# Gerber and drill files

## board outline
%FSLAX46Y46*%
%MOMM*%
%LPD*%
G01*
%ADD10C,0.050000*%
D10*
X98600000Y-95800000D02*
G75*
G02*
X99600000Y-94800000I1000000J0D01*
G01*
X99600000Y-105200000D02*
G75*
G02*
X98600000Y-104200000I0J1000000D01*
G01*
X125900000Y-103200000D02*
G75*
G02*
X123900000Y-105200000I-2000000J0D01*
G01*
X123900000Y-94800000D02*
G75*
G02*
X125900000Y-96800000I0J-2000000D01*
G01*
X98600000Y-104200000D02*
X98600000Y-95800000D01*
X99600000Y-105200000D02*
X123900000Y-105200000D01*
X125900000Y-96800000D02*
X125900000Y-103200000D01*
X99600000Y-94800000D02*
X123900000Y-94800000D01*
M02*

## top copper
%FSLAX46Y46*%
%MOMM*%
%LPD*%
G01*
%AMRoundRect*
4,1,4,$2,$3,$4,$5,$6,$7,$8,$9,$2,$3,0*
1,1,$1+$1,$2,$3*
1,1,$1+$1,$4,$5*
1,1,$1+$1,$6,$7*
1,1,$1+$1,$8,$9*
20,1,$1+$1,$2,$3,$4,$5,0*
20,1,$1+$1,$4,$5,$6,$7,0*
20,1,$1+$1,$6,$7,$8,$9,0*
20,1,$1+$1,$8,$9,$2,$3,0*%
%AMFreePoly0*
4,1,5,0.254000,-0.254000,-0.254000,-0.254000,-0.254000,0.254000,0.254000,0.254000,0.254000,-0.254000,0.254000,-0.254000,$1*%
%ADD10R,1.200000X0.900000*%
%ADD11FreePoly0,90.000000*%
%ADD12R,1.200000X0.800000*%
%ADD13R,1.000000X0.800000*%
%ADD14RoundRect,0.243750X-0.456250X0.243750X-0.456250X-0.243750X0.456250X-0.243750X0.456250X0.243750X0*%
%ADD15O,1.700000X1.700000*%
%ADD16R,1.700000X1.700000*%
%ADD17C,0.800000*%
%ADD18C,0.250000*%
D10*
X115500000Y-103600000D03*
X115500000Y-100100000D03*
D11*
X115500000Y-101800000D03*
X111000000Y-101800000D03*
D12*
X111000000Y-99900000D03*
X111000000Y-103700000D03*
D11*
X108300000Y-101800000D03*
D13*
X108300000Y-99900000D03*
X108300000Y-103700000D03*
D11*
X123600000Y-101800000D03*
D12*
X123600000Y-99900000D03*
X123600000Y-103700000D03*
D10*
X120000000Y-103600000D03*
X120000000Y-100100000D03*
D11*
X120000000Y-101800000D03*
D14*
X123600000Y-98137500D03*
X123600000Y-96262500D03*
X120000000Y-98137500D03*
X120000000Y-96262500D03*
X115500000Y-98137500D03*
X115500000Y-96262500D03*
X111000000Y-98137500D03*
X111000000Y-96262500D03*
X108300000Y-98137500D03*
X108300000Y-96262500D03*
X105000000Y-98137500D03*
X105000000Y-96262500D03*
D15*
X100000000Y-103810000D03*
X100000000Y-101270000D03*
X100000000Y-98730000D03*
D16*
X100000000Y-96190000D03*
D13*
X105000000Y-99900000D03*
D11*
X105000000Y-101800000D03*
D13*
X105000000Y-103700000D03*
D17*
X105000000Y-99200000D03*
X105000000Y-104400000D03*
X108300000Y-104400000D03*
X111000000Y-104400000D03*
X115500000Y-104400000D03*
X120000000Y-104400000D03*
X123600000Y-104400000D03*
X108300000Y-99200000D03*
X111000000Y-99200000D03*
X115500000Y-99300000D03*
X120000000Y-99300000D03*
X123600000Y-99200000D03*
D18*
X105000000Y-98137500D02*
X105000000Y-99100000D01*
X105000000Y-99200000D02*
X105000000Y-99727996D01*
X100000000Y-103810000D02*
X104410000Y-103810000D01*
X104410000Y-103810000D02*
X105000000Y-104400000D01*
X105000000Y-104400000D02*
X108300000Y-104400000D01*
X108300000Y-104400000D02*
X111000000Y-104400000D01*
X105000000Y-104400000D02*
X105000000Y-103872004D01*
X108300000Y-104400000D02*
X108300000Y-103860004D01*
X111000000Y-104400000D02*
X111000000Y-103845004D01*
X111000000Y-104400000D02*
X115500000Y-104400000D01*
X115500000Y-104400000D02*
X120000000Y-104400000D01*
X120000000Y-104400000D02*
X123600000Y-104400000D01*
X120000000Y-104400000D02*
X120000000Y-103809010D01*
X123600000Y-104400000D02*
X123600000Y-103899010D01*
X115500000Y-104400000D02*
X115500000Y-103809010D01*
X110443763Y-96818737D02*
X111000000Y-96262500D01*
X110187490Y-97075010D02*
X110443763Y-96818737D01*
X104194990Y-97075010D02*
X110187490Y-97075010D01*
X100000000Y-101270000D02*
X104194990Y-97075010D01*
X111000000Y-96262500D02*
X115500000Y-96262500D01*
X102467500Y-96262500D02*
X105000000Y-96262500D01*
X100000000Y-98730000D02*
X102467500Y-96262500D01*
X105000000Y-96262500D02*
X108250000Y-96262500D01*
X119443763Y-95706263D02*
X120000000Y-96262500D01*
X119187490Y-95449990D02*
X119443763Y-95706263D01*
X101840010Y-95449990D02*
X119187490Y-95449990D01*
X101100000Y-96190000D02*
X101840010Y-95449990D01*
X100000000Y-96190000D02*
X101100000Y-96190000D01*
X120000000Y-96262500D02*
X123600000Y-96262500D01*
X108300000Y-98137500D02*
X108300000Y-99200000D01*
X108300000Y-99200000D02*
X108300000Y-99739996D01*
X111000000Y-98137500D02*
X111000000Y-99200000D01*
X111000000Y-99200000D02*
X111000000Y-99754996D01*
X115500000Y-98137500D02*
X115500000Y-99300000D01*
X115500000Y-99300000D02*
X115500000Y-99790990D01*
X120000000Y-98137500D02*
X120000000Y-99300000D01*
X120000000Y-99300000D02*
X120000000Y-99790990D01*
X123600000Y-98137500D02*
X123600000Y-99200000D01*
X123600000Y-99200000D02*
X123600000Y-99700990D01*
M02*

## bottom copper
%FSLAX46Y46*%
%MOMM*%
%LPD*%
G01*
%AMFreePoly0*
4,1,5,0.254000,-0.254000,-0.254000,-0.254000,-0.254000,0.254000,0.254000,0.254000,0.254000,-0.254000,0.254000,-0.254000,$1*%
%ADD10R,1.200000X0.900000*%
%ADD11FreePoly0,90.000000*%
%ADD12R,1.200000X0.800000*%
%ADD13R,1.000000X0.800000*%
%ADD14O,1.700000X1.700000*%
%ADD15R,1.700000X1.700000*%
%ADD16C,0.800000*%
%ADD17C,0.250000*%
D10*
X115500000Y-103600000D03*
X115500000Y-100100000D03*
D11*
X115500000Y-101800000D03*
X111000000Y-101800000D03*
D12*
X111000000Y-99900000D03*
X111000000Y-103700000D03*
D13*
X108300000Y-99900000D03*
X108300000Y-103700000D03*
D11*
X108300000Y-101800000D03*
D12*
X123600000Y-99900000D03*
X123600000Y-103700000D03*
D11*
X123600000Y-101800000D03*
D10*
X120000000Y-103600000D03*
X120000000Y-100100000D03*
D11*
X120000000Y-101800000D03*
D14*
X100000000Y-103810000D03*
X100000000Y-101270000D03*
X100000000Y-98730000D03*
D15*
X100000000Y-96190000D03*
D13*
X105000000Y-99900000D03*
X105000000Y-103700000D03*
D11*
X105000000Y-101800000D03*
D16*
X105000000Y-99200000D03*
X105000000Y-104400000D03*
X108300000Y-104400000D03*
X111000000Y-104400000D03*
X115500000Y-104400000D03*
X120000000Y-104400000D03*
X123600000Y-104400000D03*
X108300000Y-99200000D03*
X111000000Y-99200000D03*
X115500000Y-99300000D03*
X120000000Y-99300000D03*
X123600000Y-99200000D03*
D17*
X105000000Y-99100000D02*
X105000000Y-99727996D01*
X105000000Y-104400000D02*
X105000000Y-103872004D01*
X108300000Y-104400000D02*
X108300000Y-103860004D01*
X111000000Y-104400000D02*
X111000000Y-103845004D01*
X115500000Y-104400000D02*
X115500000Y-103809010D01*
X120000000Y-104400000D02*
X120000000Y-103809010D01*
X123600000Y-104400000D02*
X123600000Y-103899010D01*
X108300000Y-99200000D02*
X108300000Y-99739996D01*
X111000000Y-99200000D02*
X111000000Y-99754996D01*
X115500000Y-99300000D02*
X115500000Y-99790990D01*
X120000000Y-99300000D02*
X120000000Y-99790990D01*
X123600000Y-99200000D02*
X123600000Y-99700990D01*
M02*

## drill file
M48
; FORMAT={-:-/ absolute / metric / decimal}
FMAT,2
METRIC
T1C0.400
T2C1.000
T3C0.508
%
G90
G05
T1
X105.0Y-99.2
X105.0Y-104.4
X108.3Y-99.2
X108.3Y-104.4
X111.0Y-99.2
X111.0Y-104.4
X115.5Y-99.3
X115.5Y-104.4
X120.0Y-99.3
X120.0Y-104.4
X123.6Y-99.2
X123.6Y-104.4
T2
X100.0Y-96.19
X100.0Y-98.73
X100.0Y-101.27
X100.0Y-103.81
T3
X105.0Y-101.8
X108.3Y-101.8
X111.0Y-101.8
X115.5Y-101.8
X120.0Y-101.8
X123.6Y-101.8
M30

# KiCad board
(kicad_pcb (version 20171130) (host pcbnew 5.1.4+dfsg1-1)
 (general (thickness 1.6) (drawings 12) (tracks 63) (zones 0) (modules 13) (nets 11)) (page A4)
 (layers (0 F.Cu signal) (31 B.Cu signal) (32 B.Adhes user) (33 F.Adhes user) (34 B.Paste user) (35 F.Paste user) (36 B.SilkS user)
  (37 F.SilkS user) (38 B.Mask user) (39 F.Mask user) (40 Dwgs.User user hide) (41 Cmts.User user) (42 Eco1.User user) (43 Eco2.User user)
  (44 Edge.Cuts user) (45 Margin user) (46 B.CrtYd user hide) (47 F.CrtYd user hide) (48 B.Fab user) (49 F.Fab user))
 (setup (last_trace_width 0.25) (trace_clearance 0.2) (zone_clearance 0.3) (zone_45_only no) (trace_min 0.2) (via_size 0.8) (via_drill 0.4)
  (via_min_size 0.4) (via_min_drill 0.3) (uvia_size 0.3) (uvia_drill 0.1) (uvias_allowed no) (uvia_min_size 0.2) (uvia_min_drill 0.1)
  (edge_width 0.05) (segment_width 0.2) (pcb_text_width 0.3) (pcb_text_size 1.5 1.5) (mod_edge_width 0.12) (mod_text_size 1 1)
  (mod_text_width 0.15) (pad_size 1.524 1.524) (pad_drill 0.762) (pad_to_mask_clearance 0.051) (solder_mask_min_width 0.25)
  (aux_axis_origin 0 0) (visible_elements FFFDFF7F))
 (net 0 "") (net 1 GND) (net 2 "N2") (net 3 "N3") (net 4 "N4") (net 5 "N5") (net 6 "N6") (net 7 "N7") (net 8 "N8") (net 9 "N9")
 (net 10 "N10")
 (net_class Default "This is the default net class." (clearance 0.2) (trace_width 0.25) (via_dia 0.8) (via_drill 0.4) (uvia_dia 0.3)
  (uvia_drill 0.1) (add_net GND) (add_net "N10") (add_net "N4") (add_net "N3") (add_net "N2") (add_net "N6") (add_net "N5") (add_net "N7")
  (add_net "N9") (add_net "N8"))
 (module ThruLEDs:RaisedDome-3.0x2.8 (layer F.Cu) (at 115.5 101.8 90)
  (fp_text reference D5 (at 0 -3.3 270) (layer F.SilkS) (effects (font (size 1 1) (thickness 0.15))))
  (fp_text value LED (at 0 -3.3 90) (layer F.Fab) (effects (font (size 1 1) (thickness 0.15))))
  (pad 1 smd rect (at -1.8 0 90) (size 0.9 1.2) (layers F.Cu F.Paste F.Mask) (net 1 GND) (zone_connect 0))
  (pad 2 smd rect (at 1.7 0 90) (size 0.9 1.2) (layers F.Cu F.Paste F.Mask) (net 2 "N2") (zone_connect 0))
  (pad 1 smd rect (at -1.8 0 90) (size 0.9 1.2) (layers B.Cu B.Paste B.Mask) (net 1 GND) (zone_connect 0))
  (pad 2 smd rect (at 1.7 0 90) (size 0.9 1.2) (layers B.Cu B.Paste B.Mask) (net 2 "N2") (zone_connect 0))
  (pad "" np_thru_hole custom (at 0 0 90) (size 0.508 0.508) (drill 0.508) (layers *.Cu *.Mask) (zone_connect 0)
   (options (clearance outline) (anchor rect)) (primitives)))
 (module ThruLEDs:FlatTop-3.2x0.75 (layer F.Cu) (at 111 101.8 90)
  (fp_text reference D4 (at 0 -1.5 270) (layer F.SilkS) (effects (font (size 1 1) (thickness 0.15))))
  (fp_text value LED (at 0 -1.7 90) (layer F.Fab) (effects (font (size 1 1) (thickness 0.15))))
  (pad "" np_thru_hole custom (at 0 0 90) (size 0.508 0.508) (drill 0.508) (layers *.Cu *.Mask) (zone_connect 0)
   (options (clearance outline) (anchor rect)) (primitives))
  (pad 2 smd rect (at 1.9 0 90) (size 0.8 1.2) (layers B.Cu B.Paste B.Mask) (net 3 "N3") (zone_connect 0))
  (pad 1 smd rect (at -1.9 0 90) (size 0.8 1.2) (layers B.Cu B.Adhes B.Mask) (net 1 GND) (zone_connect 0))
  (pad 2 smd rect (at 1.9 0 90) (size 0.8 1.2) (layers F.Cu F.Paste F.Mask) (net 3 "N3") (zone_connect 0))
  (pad 1 smd rect (at -1.9 0 90) (size 0.8 1.2) (layers F.Cu F.Paste F.Mask) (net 1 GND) (zone_connect 0)))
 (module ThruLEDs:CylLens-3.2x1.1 (layer F.Cu) (at 108.3 101.8 90)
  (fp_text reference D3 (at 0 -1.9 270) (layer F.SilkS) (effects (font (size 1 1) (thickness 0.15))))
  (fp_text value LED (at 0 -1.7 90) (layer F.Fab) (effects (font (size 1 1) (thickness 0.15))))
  (pad 2 smd rect (at 1.9 0 90) (size 0.8 1) (layers B.Cu B.Paste B.Mask) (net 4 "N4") (zone_connect 0))
  (pad 1 smd rect (at -1.9 0 90) (size 0.8 1) (layers B.Cu B.Paste B.Mask) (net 1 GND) (zone_connect 0))
  (pad "" np_thru_hole custom (at 0 0 90) (size 0.508 0.508) (drill 0.508) (layers *.Cu *.Mask) (zone_connect 0)
   (options (clearance outline) (anchor rect)) (primitives))
  (pad 2 smd rect (at 1.9 0 90) (size 0.8 1) (layers F.Cu F.Paste F.Mask) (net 4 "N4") (zone_connect 0))
  (pad 1 smd rect (at -1.9 0 90) (size 0.8 1) (layers F.Cu F.Paste F.Mask) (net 1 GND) (zone_connect 0)))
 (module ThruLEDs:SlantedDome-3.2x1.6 (layer F.Cu) (at 123.6 101.8 90)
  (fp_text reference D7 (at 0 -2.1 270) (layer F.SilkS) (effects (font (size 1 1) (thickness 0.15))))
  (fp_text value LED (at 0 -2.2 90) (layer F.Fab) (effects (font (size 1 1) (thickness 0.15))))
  (pad 2 smd rect (at 1.9 0 90) (size 0.8 1.2) (layers B.Cu B.Paste B.Mask) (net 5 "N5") (zone_connect 0))
  (pad 1 smd rect (at -1.9 0 90) (size 0.8 1.2) (layers B.Cu B.Paste B.Mask) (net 1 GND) (zone_connect 0))
  (pad "" np_thru_hole custom (at 0 0 90) (size 0.508 0.508) (drill 0.508) (layers *.Cu *.Mask) (zone_connect 0)
   (options (clearance outline) (anchor rect)) (primitives))
  (pad 2 smd rect (at 1.9 0 90) (size 0.8 1.2) (layers F.Cu F.Paste F.Mask) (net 5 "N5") (zone_connect 0))
  (pad 1 smd rect (at -1.9 0 90) (size 0.8 1.2) (layers F.Cu F.Paste F.Mask) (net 1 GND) (zone_connect 0)))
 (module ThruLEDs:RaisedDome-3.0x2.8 (layer F.Cu) (at 120 101.8 90)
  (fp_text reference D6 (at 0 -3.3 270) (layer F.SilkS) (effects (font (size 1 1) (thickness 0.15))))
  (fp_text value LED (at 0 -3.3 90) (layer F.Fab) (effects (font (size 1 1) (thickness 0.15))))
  (pad 1 smd rect (at -1.8 0 90) (size 0.9 1.2) (layers F.Cu F.Paste F.Mask) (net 1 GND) (zone_connect 0))
  (pad 2 smd rect (at 1.7 0 90) (size 0.9 1.2) (layers F.Cu F.Paste F.Mask) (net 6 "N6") (zone_connect 0))
  (pad 1 smd rect (at -1.8 0 90) (size 0.9 1.2) (layers B.Cu B.Paste B.Mask) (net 1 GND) (zone_connect 0))
  (pad 2 smd rect (at 1.7 0 90) (size 0.9 1.2) (layers B.Cu B.Paste B.Mask) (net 6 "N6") (zone_connect 0))
  (pad "" np_thru_hole custom (at 0 0 90) (size 0.508 0.508) (drill 0.508) (layers *.Cu *.Mask) (zone_connect 0)
   (options (clearance outline) (anchor rect)) (primitives)))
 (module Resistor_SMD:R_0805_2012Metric (layer F.Cu) (at 123.6 97.2 270)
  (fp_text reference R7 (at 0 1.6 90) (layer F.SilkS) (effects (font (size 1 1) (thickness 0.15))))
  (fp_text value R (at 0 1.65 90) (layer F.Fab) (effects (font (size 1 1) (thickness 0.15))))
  (pad 2 smd roundrect (at 0.9375 0 270) (size 0.975 1.4) (layers F.Cu F.Paste F.Mask) (roundrect_rratio 0.25) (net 5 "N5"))
  (pad 1 smd roundrect (at -0.9375 0 270) (size 0.975 1.4) (layers F.Cu F.Paste F.Mask) (roundrect_rratio 0.25) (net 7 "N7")))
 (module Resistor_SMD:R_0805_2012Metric (layer F.Cu) (at 120 97.2 270)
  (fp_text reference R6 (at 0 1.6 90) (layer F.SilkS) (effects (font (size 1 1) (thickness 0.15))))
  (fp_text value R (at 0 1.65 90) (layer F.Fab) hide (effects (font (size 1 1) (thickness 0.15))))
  (pad 2 smd roundrect (at 0.9375 0 270) (size 0.975 1.4) (layers F.Cu F.Paste F.Mask) (roundrect_rratio 0.25) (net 6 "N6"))
  (pad 1 smd roundrect (at -0.9375 0 270) (size 0.975 1.4) (layers F.Cu F.Paste F.Mask) (roundrect_rratio 0.25) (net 7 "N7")))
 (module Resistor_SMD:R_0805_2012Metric (layer F.Cu) (at 115.5 97.2 270)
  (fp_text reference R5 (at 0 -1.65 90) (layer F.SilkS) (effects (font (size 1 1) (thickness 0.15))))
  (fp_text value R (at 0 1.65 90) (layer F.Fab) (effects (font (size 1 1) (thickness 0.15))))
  (pad 2 smd roundrect (at 0.9375 0 270) (size 0.975 1.4) (layers F.Cu F.Paste F.Mask) (roundrect_rratio 0.25) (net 2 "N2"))
  (pad 1 smd roundrect (at -0.9375 0 270) (size 0.975 1.4) (layers F.Cu F.Paste F.Mask) (roundrect_rratio 0.25) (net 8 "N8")))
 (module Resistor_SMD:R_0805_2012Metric (layer F.Cu) (at 111 97.2 270)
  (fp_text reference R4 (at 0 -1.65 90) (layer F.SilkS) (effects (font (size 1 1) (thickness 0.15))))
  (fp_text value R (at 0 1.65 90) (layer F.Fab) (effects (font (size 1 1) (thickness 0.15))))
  (pad 2 smd roundrect (at 0.9375 0 270) (size 0.975 1.4) (layers F.Cu F.Paste F.Mask) (roundrect_rratio 0.25) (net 3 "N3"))
  (pad 1 smd roundrect (at -0.9375 0 270) (size 0.975 1.4) (layers F.Cu F.Paste F.Mask) (roundrect_rratio 0.25) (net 8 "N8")))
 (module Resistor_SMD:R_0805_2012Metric (layer F.Cu) (at 108.3 97.2 270)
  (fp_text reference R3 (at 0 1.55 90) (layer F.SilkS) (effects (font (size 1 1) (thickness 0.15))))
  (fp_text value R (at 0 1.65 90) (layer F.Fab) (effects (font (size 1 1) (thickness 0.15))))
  (pad 2 smd roundrect (at 0.9375 0 270) (size 0.975 1.4) (layers F.Cu F.Paste F.Mask) (roundrect_rratio 0.25) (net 4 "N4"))
  (pad 1 smd roundrect (at -0.9375 0 270) (size 0.975 1.4) (layers F.Cu F.Paste F.Mask) (roundrect_rratio 0.25) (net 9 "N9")))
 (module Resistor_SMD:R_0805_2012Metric (layer F.Cu) (at 105 97.2 270)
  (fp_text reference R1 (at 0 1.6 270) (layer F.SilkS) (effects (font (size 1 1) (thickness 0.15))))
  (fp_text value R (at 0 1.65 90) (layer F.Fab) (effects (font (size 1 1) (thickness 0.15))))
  (pad 2 smd roundrect (at 0.9375 0 270) (size 0.975 1.4) (layers F.Cu F.Paste F.Mask) (roundrect_rratio 0.25) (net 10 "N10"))
  (pad 1 smd roundrect (at -0.9375 0 270) (size 0.975 1.4) (layers F.Cu F.Paste F.Mask) (roundrect_rratio 0.25) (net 9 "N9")))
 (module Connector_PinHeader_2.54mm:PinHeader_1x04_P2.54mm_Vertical (layer B.Cu) (at 100 96.19 180)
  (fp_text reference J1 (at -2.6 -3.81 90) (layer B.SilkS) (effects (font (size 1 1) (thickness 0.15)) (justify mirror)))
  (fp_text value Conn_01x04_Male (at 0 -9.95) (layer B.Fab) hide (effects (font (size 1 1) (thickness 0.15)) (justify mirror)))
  (pad 4 thru_hole oval (at 0 -7.62 180) (size 1.7 1.7) (drill 1) (layers *.Cu *.Mask) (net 1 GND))
  (pad 3 thru_hole oval (at 0 -5.08 180) (size 1.7 1.7) (drill 1) (layers *.Cu *.Mask) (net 8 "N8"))
  (pad 2 thru_hole oval (at 0 -2.54 180) (size 1.7 1.7) (drill 1) (layers *.Cu *.Mask) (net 9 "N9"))
  (pad 1 thru_hole rect (at 0 0 180) (size 1.7 1.7) (drill 1) (layers *.Cu *.Mask) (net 7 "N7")))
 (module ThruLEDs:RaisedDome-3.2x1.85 (layer F.Cu) (at 105 101.8 90)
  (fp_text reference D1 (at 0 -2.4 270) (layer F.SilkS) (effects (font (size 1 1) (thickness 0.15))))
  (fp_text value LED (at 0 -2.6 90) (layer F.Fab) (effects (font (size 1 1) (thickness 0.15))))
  (pad 2 smd rect (at 1.9 0 90) (size 0.8 1) (layers F.Cu F.Paste F.Mask) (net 10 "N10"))
  (pad 2 smd rect (at 1.9 0 90) (size 0.8 1) (layers B.Cu B.Paste B.Mask) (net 10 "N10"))
  (pad 1 smd rect (at -1.9 0 90) (size 0.8 1) (layers B.Cu B.Paste B.Mask) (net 1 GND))
  (pad "" np_thru_hole custom (at 0 0 90) (size 0.508 0.508) (drill 0.508) (layers *.Cu *.Mask) (zone_connect 0)
   (options (clearance outline) (anchor rect)) (primitives))
  (pad 1 smd rect (at -1.9 0 90) (size 0.8 1) (layers F.Cu F.Paste F.Mask) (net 1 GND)))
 (gr_arc (start 99.6 95.8) (end 98.6 95.8) (angle 90) (layer Edge.Cuts) (width 0.05))
 (gr_arc (start 99.6 104.2) (end 99.6 105.2) (angle 90) (layer Edge.Cuts) (width 0.05))
 (gr_arc (start 123.9 103.2) (end 123.9 105.2) (angle -90) (layer Edge.Cuts) (width 0.05))
 (gr_arc (start 123.9 96.8) (end 125.9 96.8) (angle -90) (layer Edge.Cuts) (width 0.05))
 (gr_line (start 98.6 104.2) (end 98.6 95.8) (layer Edge.Cuts) (width 0.05))
 (gr_line (start 99.6 105.2) (end 123.9 105.2) (layer Edge.Cuts) (width 0.05))
 (gr_line (start 125.9 96.8) (end 125.9 103.2) (layer Edge.Cuts) (width 0.05))
 (gr_line (start 99.6 94.8) (end 123.9 94.8) (layer Edge.Cuts) (width 0.05))
 (via (at 105 99.2) (size 0.8) (drill 0.4) (layers F.Cu B.Cu) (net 10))
 (segment (start 105 98.1375) (end 105 99.1) (width 0.25) (layer F.Cu) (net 10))
 (segment (start 105 99.1) (end 105 99.727996) (width 0.25) (layer B.Cu) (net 10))
 (segment (start 105 99.2) (end 105 99.727996) (width 0.25) (layer F.Cu) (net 10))
 (via (at 105 104.4) (size 0.8) (drill 0.4) (layers F.Cu B.Cu) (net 1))
 (segment (start 100 103.81) (end 104.41 103.81) (width 0.25) (layer F.Cu) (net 1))
 (segment (start 104.41 103.81) (end 105 104.4) (width 0.25) (layer F.Cu) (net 1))
 (segment (start 105 104.4) (end 105 103.872004) (width 0.25) (layer B.Cu) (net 1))
 (via (at 108.3 104.4) (size 0.8) (drill 0.4) (layers F.Cu B.Cu) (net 1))
 (segment (start 105 104.4) (end 108.3 104.4) (width 0.25) (layer F.Cu) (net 1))
 (segment (start 108.3 104.4) (end 108.3 103.860004) (width 0.25) (layer B.Cu) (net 1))
 (via (at 111 104.4) (size 0.8) (drill 0.4) (layers F.Cu B.Cu) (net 1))
 (segment (start 108.3 104.4) (end 111 104.4) (width 0.25) (layer F.Cu) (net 1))
 (segment (start 111 104.4) (end 111 103.845004) (width 0.25) (layer B.Cu) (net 1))
 (segment (start 105 104.4) (end 105 103.872004) (width 0.25) (layer F.Cu) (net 1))
 (segment (start 108.3 104.4) (end 108.3 103.860004) (width 0.25) (layer F.Cu) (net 1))
 (segment (start 111 104.4) (end 111 103.845004) (width 0.25) (layer F.Cu) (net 1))
 (via (at 115.5 104.4) (size 0.8) (drill 0.4) (layers F.Cu B.Cu) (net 1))
 (segment (start 111 104.4) (end 115.5 104.4) (width 0.25) (layer F.Cu) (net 1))
 (segment (start 115.5 104.4) (end 115.5 103.80901) (width 0.25) (layer B.Cu) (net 1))
 (via (at 120 104.4) (size 0.8) (drill 0.4) (layers F.Cu B.Cu) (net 1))
 (segment (start 115.5 104.4) (end 120 104.4) (width 0.25) (layer F.Cu) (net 1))
 (segment (start 120 104.4) (end 120 103.80901) (width 0.25) (layer B.Cu) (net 1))
 (via (at 123.6 104.4) (size 0.8) (drill 0.4) (layers F.Cu B.Cu) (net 1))
 (segment (start 120 104.4) (end 123.6 104.4) (width 0.25) (layer F.Cu) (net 1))
 (segment (start 123.6 104.4) (end 123.6 103.89901) (width 0.25) (layer B.Cu) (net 1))
 (segment (start 120 104.4) (end 120 103.80901) (width 0.25) (layer F.Cu) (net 1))
 (segment (start 123.6 104.4) (end 123.6 103.89901) (width 0.25) (layer F.Cu) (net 1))
 (segment (start 115.5 104.4) (end 115.5 103.80901) (width 0.25) (layer F.Cu) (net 1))
 (segment (start 110.443763 96.818737) (end 111 96.2625) (width 0.25) (layer F.Cu) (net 8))
 (segment (start 110.18749 97.07501) (end 110.443763 96.818737) (width 0.25) (layer F.Cu) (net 8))
 (segment (start 104.19499 97.07501) (end 110.18749 97.07501) (width 0.25) (layer F.Cu) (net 8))
 (segment (start 100 101.27) (end 104.19499 97.07501) (width 0.25) (layer F.Cu) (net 8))
 (segment (start 111 96.2625) (end 115.5 96.2625) (width 0.25) (layer F.Cu) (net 8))
 (segment (start 102.4675 96.2625) (end 105 96.2625) (width 0.25) (layer F.Cu) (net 9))
 (segment (start 100 98.73) (end 102.4675 96.2625) (width 0.25) (layer F.Cu) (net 9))
 (segment (start 105 96.2625) (end 108.25 96.2625) (width 0.25) (layer F.Cu) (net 9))
 (segment (start 119.443763 95.706263) (end 120 96.2625) (width 0.25) (layer F.Cu) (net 7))
 (segment (start 119.18749 95.44999) (end 119.443763 95.706263) (width 0.25) (layer F.Cu) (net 7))
 (segment (start 101.84001 95.44999) (end 119.18749 95.44999) (width 0.25) (layer F.Cu) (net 7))
 (segment (start 101.1 96.19) (end 101.84001 95.44999) (width 0.25) (layer F.Cu) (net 7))
 (segment (start 100 96.19) (end 101.1 96.19) (width 0.25) (layer F.Cu) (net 7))
 (segment (start 120 96.2625) (end 123.6 96.2625) (width 0.25) (layer F.Cu) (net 7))
 (via (at 108.3 99.2) (size 0.8) (drill 0.4) (layers F.Cu B.Cu) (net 4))
 (segment (start 108.3 98.1375) (end 108.3 99.2) (width 0.25) (layer F.Cu) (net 4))
 (segment (start 108.3 99.2) (end 108.3 99.739996) (width 0.25) (layer B.Cu) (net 4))
 (segment (start 108.3 99.2) (end 108.3 99.739996) (width 0.25) (layer F.Cu) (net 4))
 (via (at 111 99.2) (size 0.8) (drill 0.4) (layers F.Cu B.Cu) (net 3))
 (segment (start 111 98.1375) (end 111 99.2) (width 0.25) (layer F.Cu) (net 3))
 (segment (start 111 99.2) (end 111 99.754996) (width 0.25) (layer B.Cu) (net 3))
 (segment (start 111 99.2) (end 111 99.754996) (width 0.25) (layer F.Cu) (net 3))
 (via (at 115.5 99.3) (size 0.8) (drill 0.4) (layers F.Cu B.Cu) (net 2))
 (segment (start 115.5 98.1375) (end 115.5 99.3) (width 0.25) (layer F.Cu) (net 2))
 (segment (start 115.5 99.3) (end 115.5 99.79099) (width 0.25) (layer B.Cu) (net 2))
 (segment (start 115.5 99.3) (end 115.5 99.79099) (width 0.25) (layer F.Cu) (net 2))
 (via (at 120 99.3) (size 0.8) (drill 0.4) (layers F.Cu B.Cu) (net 6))
 (segment (start 120 98.1375) (end 120 99.3) (width 0.25) (layer F.Cu) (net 6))
 (segment (start 120 99.3) (end 120 99.79099) (width 0.25) (layer B.Cu) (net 6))
 (segment (start 120 99.3) (end 120 99.79099) (width 0.25) (layer F.Cu) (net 6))
 (via (at 123.6 99.2) (size 0.8) (drill 0.4) (layers F.Cu B.Cu) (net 5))
 (segment (start 123.6 98.1375) (end 123.6 99.2) (width 0.25) (layer F.Cu) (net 5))
 (segment (start 123.6 99.2) (end 123.6 99.70099) (width 0.25) (layer B.Cu) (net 5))
 (segment (start 123.6 99.2) (end 123.6 99.70099) (width 0.25) (layer F.Cu) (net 5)))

